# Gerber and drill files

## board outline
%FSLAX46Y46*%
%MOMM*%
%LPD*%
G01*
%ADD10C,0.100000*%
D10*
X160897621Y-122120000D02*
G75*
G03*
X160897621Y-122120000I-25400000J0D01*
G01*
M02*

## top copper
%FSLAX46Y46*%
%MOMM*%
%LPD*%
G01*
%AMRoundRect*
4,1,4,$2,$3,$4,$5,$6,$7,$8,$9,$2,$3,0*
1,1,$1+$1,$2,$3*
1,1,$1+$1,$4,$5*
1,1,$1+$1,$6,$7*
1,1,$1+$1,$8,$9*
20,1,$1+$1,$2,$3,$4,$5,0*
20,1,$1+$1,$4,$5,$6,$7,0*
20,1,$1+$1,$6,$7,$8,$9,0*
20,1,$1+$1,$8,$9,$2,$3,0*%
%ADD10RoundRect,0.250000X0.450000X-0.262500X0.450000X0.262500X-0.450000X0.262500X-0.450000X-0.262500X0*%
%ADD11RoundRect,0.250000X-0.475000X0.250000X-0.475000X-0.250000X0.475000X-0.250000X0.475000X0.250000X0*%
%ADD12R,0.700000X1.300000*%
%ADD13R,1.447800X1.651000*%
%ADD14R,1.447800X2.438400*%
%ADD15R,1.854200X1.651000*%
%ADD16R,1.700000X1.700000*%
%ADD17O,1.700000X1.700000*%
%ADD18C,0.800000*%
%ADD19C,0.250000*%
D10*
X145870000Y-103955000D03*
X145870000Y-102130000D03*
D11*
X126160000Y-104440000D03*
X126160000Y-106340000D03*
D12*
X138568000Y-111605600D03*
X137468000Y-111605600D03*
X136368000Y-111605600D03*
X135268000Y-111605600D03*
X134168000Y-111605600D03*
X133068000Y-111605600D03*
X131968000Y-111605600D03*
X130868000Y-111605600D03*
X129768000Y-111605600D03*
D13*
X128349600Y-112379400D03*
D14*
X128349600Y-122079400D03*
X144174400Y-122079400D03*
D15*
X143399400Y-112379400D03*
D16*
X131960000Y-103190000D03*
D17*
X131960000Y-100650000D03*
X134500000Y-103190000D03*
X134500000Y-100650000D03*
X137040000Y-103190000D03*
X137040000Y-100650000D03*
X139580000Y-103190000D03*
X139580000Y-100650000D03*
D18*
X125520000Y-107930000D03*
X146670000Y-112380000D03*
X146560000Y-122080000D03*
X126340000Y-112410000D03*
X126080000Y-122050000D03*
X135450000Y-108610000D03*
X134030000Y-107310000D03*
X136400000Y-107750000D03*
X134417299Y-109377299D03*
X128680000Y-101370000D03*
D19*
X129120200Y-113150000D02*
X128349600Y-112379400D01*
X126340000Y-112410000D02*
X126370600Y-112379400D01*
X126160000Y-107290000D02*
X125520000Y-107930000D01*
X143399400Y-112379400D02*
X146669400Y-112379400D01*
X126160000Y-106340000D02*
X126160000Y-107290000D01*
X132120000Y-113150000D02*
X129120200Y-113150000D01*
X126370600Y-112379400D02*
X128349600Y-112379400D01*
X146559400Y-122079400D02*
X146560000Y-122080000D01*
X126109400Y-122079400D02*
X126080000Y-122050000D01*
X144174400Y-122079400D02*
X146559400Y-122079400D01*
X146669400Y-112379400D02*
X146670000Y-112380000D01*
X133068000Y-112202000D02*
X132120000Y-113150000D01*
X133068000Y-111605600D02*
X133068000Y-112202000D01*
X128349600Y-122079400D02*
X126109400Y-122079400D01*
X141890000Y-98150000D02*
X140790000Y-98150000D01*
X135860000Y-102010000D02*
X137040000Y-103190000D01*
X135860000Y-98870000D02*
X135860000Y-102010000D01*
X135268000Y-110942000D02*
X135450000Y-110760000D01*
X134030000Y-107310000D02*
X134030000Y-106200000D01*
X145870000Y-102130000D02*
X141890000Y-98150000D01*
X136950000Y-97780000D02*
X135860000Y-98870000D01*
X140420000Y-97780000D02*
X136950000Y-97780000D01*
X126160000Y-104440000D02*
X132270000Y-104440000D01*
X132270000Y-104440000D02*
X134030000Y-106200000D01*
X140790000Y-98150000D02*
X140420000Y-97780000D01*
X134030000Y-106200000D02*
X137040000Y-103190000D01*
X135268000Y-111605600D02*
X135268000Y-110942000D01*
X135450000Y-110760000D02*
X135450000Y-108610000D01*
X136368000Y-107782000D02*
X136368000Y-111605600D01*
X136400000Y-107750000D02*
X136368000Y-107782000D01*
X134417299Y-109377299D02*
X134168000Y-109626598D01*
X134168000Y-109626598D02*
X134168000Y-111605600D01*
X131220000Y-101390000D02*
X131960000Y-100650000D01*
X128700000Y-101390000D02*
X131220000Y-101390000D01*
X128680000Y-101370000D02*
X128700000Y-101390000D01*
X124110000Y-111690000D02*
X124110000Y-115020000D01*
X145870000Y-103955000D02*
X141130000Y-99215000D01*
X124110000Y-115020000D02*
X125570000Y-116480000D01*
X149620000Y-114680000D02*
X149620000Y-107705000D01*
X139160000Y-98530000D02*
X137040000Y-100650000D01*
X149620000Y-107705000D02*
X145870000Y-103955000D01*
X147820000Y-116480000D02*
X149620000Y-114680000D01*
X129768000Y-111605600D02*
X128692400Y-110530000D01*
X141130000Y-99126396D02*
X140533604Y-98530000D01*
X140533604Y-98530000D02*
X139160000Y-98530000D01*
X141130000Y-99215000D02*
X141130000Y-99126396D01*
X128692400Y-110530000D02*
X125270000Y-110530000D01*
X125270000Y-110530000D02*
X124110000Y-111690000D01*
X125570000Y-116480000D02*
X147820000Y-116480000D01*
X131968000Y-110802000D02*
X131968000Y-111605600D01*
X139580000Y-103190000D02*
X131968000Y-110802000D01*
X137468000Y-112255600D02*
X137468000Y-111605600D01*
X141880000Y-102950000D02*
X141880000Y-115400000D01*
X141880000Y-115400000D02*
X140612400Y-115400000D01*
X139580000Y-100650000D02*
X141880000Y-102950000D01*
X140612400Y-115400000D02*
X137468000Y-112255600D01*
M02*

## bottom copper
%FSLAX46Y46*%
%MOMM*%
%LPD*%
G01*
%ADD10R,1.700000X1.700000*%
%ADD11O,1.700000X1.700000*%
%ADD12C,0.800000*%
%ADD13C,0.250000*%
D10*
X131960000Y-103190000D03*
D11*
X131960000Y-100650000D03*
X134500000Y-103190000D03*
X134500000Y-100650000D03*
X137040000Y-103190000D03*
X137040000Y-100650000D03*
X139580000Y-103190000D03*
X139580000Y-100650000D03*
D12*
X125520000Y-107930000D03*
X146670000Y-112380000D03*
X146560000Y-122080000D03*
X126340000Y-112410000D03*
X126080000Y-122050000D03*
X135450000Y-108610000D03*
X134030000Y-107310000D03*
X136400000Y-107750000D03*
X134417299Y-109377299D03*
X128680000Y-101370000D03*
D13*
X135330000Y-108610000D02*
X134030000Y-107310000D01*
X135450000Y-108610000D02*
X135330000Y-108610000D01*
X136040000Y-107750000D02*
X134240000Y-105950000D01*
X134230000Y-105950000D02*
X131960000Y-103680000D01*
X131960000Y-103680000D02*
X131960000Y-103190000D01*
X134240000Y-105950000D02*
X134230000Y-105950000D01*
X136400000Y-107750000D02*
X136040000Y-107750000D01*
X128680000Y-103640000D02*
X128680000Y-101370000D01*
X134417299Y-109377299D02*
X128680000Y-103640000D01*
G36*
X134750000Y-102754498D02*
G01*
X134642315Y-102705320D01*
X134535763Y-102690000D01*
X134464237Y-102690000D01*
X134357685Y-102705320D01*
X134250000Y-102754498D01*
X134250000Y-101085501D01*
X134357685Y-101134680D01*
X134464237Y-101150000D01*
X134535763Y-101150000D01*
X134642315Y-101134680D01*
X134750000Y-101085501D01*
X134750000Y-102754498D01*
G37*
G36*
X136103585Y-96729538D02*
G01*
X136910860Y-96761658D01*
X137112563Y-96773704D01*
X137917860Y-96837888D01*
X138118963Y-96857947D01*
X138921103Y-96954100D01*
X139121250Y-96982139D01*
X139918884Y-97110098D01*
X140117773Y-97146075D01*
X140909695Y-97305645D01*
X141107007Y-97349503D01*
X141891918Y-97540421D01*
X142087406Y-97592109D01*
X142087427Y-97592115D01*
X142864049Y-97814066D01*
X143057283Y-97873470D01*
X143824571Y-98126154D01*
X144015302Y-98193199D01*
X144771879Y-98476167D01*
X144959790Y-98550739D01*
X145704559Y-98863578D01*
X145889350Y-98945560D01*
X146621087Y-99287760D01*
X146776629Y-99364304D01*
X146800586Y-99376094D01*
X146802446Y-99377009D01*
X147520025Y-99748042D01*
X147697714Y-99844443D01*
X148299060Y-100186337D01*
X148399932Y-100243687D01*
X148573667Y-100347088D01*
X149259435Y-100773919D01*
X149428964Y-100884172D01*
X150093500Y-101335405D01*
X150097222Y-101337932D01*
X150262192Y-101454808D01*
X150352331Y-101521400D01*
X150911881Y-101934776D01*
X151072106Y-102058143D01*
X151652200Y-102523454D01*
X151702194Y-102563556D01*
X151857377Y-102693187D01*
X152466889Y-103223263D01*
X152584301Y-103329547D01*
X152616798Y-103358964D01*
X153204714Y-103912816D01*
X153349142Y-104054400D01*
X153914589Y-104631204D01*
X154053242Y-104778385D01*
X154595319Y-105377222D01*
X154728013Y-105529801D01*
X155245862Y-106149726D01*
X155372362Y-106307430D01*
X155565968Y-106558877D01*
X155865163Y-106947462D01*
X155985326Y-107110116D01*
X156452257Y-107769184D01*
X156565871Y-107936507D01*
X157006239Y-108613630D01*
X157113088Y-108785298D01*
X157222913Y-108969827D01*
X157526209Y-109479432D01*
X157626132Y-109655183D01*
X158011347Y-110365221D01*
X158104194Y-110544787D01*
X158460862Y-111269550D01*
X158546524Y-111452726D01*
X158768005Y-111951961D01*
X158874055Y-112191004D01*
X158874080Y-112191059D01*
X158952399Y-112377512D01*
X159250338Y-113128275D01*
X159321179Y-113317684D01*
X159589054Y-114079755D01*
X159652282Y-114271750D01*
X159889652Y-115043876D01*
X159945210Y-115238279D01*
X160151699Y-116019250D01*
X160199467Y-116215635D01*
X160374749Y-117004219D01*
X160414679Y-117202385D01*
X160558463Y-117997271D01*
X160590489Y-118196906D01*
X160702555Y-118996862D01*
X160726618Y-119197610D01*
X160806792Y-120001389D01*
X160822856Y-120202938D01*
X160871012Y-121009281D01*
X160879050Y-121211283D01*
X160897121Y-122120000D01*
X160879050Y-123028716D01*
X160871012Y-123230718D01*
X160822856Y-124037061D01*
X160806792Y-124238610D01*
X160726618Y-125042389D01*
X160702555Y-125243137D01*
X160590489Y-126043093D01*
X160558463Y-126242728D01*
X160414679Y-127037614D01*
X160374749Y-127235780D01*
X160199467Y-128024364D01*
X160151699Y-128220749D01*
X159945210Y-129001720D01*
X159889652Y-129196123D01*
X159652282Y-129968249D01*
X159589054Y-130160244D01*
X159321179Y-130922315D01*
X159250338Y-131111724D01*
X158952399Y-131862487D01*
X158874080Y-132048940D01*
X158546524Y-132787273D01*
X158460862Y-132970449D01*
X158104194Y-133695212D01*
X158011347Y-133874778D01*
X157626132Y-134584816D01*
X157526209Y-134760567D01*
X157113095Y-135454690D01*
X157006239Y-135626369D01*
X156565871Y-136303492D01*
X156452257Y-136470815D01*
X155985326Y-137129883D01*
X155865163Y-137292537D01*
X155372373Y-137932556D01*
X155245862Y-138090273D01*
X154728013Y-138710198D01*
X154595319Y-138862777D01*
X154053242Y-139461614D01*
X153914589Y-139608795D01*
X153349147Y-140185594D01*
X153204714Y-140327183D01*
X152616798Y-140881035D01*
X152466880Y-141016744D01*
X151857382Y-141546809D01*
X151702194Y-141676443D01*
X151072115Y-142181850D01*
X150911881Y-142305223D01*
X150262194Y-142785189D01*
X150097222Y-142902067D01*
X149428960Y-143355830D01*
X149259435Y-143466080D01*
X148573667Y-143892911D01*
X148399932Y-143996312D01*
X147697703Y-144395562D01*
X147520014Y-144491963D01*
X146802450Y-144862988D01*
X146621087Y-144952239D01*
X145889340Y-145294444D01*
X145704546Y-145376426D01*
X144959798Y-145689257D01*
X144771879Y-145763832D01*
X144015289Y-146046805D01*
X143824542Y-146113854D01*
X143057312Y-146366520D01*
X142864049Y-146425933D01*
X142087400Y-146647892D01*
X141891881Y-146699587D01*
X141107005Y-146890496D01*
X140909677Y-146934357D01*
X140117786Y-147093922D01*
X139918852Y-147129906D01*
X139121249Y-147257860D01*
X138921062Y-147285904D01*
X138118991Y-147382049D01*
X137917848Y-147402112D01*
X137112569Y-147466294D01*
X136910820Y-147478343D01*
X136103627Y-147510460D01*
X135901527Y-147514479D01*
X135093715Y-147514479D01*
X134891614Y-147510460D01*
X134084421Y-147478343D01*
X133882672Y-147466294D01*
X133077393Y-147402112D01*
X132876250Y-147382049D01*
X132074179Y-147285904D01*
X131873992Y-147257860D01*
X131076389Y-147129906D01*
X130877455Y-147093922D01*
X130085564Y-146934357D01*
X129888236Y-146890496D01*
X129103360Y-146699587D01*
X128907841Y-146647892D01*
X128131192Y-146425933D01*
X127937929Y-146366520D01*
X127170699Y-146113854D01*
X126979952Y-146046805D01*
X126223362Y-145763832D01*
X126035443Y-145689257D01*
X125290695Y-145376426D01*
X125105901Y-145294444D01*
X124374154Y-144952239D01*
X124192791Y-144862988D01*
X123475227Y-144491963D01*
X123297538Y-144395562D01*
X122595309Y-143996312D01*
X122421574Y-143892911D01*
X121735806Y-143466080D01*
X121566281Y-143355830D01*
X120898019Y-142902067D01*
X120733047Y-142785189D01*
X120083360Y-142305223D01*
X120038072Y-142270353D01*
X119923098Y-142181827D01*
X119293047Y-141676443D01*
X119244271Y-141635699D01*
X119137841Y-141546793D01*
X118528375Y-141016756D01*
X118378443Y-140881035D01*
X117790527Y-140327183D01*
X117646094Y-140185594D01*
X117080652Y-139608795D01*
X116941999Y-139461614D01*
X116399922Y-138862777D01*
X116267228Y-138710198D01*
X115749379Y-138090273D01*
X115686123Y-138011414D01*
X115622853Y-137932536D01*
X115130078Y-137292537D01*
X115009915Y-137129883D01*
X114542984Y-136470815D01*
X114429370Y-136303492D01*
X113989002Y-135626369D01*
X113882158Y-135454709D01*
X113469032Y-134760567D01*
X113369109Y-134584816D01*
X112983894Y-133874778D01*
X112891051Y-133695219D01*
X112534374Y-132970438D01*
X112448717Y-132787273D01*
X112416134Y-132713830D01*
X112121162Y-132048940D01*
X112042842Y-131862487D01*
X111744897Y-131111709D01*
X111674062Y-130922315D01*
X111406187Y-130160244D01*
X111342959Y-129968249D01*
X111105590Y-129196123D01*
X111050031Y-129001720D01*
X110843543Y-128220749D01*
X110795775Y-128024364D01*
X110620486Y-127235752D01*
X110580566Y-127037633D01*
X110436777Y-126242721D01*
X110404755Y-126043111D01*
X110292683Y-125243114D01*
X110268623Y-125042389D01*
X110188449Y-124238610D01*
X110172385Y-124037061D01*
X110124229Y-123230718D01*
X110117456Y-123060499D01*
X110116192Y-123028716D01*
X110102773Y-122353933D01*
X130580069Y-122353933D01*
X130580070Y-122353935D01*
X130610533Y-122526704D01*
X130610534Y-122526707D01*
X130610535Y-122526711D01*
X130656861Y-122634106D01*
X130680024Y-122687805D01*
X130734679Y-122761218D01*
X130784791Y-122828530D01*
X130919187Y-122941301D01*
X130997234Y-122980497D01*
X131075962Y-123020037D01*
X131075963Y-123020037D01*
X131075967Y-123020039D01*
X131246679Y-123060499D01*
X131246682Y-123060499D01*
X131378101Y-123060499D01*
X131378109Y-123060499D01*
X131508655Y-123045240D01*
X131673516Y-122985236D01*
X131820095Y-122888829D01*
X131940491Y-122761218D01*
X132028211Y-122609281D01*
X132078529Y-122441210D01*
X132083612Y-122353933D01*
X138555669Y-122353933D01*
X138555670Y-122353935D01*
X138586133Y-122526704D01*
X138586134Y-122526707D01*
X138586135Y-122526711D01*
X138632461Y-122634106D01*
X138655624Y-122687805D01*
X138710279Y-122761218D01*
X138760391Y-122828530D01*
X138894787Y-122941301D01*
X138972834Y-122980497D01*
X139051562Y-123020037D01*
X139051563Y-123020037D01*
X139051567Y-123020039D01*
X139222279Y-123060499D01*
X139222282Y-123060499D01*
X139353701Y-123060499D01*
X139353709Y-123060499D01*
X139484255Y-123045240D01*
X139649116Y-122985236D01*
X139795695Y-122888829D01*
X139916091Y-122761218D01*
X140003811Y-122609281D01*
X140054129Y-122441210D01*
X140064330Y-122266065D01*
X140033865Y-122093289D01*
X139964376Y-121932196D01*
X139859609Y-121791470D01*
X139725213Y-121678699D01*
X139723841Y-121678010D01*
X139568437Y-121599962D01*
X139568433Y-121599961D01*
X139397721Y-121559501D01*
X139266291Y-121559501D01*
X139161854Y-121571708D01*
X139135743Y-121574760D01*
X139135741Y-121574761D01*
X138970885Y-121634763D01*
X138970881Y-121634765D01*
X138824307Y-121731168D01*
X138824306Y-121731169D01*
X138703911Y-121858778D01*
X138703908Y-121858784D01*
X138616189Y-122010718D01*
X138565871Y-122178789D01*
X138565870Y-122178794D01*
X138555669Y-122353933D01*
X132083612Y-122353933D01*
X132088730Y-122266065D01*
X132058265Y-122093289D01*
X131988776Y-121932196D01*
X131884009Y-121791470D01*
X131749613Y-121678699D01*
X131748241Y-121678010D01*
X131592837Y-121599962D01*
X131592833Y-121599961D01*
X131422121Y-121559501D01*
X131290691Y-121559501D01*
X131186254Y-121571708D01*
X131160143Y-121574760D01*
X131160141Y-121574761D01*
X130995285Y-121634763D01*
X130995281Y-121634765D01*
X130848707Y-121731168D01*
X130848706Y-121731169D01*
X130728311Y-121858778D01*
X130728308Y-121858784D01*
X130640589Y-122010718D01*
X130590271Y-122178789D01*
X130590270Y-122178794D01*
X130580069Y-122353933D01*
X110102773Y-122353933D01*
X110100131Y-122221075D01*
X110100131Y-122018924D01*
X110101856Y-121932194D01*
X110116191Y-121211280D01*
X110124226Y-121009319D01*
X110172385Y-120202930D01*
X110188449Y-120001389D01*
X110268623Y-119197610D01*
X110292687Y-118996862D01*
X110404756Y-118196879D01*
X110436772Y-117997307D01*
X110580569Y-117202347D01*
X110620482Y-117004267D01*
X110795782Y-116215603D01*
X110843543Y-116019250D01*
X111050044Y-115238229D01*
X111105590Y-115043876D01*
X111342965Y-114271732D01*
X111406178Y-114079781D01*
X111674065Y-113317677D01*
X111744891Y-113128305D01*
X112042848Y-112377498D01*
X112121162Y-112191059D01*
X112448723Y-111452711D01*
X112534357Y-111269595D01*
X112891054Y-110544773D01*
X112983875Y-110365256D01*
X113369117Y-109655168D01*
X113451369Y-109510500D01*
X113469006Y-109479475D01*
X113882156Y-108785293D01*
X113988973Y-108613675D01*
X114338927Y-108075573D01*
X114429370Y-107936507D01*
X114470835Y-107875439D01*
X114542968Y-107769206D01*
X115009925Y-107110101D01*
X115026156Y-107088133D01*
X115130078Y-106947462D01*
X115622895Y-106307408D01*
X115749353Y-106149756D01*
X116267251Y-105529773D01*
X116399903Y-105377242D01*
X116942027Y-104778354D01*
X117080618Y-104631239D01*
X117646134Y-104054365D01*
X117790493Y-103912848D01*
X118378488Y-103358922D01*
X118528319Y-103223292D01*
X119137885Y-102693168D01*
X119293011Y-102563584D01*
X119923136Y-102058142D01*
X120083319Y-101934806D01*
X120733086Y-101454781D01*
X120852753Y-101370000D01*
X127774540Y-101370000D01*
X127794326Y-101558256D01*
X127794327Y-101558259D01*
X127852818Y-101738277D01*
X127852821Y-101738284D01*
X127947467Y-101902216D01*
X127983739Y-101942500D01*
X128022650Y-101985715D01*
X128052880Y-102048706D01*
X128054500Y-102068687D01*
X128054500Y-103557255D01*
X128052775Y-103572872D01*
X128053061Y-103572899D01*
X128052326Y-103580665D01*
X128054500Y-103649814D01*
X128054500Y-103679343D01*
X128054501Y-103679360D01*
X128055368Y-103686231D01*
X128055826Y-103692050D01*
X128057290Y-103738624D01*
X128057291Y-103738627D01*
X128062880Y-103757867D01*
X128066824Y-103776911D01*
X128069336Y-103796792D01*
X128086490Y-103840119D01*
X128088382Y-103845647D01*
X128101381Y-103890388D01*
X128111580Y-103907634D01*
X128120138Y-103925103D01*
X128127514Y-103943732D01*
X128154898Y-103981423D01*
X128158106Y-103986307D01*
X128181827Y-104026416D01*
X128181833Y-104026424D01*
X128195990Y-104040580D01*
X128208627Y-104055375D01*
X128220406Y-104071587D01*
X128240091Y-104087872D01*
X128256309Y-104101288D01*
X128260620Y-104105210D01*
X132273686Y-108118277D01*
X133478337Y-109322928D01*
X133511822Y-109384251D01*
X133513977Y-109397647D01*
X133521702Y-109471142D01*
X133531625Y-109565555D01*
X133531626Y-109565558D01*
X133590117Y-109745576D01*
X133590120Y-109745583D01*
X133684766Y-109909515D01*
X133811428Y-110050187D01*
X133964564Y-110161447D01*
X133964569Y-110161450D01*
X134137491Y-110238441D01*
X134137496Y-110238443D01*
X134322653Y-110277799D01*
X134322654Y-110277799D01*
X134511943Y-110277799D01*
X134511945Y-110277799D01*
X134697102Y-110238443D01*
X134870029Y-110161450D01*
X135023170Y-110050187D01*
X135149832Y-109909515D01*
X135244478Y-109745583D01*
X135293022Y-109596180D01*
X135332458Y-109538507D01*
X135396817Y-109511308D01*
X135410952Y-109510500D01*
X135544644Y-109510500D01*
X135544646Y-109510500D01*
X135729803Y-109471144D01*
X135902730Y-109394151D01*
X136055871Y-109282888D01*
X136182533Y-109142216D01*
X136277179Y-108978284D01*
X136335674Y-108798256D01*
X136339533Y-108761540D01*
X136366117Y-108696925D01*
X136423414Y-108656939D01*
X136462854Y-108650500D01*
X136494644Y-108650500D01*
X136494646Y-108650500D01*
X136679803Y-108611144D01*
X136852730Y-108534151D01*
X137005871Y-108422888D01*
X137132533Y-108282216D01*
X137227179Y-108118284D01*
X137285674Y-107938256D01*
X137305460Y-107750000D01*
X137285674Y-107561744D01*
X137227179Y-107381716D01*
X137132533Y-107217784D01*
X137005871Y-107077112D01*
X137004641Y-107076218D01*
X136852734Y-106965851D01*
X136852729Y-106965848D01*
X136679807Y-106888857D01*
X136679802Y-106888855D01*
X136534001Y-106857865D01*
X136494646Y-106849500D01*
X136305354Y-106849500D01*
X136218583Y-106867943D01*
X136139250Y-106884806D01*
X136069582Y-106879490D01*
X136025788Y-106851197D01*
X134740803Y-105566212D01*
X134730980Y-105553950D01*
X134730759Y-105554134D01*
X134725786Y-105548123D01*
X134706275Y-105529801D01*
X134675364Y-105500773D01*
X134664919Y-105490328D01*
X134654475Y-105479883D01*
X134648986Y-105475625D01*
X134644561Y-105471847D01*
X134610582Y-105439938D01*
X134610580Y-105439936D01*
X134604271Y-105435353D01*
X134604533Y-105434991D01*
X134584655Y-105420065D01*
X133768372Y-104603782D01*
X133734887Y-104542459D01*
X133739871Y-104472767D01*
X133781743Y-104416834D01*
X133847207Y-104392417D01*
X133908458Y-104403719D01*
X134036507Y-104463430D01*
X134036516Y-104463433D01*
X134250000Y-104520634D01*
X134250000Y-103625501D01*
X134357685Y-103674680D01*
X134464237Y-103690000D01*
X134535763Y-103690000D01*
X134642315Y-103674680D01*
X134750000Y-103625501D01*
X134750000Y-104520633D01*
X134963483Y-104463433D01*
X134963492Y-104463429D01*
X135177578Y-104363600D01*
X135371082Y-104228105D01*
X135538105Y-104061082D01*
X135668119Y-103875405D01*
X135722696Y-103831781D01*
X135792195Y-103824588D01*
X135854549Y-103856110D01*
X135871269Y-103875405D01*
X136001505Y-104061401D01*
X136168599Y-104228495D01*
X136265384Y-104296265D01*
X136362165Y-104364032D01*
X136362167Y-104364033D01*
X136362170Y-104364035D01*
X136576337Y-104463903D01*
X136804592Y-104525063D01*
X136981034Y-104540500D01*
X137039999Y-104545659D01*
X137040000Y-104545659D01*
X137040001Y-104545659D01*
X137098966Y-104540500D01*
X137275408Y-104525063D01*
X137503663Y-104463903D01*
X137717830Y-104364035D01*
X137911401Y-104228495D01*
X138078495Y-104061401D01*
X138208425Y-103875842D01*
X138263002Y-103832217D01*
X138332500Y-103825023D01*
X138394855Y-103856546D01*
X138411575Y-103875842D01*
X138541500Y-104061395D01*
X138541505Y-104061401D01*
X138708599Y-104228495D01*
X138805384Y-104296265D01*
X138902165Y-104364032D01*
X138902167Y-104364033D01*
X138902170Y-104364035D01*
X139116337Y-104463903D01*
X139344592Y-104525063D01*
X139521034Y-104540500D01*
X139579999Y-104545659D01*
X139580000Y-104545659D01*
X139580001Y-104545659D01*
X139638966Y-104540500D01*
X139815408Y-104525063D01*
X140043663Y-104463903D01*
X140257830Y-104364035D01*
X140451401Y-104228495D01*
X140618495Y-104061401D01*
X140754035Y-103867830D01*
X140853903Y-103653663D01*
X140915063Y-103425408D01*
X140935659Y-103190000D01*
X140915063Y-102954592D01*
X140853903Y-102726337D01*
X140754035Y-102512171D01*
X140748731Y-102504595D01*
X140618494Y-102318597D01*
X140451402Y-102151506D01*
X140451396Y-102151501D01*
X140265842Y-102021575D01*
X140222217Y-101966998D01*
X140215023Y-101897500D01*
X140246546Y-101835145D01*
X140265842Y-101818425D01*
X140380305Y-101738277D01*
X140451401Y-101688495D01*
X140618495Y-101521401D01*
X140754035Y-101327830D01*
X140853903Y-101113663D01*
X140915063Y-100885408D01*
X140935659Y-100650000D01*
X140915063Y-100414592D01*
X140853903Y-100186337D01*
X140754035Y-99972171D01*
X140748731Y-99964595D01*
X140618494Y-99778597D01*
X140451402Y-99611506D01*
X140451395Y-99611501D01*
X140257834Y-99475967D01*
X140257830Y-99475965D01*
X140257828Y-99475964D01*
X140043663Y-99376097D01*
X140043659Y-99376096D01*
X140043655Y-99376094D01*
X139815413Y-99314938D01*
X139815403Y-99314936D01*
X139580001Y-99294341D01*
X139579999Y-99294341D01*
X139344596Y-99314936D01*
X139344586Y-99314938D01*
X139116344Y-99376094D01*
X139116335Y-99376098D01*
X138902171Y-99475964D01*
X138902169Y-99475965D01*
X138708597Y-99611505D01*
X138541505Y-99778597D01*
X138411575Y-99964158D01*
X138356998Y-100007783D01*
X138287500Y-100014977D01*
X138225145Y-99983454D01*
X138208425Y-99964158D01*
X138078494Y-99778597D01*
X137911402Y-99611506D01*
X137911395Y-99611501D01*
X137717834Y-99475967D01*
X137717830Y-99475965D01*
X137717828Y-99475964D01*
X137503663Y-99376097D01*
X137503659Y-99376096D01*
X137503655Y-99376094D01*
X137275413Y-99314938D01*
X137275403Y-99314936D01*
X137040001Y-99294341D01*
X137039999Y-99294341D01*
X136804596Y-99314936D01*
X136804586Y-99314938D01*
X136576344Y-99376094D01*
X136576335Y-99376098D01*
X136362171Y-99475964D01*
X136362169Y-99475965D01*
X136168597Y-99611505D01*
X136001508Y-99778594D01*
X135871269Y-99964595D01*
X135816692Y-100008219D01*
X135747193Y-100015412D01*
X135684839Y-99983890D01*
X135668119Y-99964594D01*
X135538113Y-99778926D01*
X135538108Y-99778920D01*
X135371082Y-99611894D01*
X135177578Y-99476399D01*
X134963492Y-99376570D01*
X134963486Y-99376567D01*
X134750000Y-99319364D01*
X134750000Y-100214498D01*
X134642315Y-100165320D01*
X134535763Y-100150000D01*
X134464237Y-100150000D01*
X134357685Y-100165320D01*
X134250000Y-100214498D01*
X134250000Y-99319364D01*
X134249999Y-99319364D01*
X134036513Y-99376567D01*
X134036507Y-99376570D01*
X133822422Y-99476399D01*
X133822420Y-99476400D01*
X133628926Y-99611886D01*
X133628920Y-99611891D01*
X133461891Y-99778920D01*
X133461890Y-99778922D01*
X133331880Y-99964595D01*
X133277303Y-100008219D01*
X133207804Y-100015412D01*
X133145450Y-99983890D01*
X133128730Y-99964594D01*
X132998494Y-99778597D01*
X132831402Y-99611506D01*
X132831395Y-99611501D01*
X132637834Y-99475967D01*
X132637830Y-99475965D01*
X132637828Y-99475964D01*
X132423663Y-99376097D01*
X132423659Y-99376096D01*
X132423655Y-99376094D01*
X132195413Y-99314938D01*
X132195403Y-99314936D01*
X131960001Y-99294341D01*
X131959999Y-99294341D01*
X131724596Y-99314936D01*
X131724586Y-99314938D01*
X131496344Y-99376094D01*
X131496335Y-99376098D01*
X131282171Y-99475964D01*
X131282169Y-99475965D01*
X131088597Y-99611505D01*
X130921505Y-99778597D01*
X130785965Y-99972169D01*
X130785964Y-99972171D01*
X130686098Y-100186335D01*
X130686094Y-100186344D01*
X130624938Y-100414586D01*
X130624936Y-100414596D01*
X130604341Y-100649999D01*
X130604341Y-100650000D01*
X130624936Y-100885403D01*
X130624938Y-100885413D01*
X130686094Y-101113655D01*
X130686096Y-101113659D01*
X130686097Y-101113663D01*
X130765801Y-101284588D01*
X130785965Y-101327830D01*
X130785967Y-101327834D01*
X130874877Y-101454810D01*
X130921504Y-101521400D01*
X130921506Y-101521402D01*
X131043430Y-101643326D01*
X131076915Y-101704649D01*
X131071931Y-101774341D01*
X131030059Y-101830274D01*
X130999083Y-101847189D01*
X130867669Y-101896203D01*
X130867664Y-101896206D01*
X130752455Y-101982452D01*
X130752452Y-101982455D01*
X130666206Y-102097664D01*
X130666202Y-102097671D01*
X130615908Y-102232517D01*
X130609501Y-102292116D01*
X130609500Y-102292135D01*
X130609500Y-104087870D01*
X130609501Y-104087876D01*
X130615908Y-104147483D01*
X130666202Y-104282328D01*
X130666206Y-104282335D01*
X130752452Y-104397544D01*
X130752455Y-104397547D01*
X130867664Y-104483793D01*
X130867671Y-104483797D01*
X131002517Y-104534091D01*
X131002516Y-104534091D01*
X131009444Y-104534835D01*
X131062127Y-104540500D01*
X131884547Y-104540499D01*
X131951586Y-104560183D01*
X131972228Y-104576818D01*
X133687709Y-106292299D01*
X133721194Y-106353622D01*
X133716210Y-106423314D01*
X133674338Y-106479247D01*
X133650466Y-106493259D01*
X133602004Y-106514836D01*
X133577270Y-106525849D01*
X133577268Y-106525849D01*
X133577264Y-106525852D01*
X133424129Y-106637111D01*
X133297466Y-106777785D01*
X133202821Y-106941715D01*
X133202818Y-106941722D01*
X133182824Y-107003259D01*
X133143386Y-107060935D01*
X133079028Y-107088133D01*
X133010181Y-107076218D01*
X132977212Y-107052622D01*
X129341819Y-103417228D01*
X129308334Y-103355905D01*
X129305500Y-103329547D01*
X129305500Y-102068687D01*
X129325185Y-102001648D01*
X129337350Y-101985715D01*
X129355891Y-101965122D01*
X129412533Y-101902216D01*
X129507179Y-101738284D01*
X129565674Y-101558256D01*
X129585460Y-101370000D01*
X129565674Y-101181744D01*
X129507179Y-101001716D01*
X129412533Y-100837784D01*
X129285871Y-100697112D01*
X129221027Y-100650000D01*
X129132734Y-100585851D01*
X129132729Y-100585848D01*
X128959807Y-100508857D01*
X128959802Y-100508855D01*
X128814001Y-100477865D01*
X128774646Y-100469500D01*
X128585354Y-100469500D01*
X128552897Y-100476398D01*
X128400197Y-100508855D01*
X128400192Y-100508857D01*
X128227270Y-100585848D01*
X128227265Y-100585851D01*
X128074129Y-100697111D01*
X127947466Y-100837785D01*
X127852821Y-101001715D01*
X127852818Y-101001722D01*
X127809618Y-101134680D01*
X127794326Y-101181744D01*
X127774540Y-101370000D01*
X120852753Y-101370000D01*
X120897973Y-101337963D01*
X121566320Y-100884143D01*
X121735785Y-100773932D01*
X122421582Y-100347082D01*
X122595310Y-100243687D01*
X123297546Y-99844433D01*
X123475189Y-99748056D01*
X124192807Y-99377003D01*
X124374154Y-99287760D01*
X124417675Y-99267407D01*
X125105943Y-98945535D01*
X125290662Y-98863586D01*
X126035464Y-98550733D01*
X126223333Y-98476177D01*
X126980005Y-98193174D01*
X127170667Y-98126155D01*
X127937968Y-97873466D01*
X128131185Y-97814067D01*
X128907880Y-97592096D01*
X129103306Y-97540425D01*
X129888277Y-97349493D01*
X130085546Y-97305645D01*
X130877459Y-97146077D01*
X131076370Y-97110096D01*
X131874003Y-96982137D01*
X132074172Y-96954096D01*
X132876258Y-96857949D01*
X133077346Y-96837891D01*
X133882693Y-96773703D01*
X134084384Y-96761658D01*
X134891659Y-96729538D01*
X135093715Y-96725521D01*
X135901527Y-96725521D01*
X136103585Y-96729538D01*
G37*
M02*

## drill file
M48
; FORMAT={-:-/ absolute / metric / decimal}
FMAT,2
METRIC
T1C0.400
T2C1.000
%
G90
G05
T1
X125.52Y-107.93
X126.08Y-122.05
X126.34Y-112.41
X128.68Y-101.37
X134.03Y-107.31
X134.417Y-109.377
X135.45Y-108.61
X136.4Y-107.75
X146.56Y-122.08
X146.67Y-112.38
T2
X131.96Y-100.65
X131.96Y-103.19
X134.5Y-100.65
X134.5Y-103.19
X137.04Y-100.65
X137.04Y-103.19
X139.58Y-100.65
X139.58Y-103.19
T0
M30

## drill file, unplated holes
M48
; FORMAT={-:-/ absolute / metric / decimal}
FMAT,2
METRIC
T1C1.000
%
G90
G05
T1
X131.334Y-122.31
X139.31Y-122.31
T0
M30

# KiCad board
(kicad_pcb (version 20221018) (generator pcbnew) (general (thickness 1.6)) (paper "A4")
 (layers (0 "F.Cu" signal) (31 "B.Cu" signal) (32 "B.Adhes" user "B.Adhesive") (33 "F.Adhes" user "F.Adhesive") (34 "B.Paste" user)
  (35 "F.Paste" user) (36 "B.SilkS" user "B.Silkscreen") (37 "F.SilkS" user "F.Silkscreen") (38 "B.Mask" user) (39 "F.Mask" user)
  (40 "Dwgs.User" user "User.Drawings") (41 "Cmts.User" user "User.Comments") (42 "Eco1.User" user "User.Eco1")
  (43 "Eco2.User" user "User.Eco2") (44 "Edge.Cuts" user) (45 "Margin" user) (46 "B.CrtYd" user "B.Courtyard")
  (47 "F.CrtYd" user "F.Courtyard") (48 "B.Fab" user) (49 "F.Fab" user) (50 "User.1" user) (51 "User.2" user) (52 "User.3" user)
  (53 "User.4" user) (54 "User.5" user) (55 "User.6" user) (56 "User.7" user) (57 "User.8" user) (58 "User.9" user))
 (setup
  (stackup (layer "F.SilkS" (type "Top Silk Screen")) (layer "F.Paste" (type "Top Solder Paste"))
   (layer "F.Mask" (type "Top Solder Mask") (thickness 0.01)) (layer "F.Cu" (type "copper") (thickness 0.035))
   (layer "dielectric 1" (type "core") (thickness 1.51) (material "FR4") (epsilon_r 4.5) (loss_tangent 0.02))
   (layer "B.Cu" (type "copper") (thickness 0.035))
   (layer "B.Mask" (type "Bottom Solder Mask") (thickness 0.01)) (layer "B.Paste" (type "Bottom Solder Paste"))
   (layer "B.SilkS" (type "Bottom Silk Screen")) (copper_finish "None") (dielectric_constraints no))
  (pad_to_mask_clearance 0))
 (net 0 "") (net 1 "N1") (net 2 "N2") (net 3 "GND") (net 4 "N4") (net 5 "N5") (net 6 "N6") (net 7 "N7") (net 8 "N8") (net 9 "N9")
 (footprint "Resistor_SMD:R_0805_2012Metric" (layer "F.Cu") (at 145.87 103.0425 90)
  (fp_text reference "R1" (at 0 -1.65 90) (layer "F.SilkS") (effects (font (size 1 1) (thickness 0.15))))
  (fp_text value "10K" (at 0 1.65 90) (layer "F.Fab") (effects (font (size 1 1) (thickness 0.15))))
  (pad "1" smd roundrect (at -0.9125 0 90) (size 1.025 1.4) (layers "F.Cu" "F.Paste" "F.Mask") (roundrect_rratio 0.243902439) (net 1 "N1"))
  (pad "2" smd roundrect (at 0.9125 0 90) (size 1.025 1.4) (layers "F.Cu" "F.Paste" "F.Mask") (roundrect_rratio 0.243902439) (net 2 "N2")))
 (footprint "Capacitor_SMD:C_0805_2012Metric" (layer "F.Cu") (at 126.16 105.39 -90)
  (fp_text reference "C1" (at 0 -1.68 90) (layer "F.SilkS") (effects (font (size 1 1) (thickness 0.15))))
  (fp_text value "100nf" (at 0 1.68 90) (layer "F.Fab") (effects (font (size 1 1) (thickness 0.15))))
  (pad "1" smd roundrect (at -0.95 0 270) (size 1 1.45) (layers "F.Cu" "F.Paste" "F.Mask") (roundrect_rratio 0.25) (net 2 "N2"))
  (pad "2" smd roundrect (at 0.95 0 270) (size 1 1.45) (layers "F.Cu" "F.Paste" "F.Mask") (roundrect_rratio 0.25) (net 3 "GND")))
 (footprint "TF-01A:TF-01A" (layer "F.Cu") (at 136.3382 118.7794)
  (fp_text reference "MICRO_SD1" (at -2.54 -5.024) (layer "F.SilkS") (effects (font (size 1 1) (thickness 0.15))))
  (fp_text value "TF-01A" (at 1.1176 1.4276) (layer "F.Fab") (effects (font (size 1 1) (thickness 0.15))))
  (pad "" np_thru_hole circle (at -5.0038 3.5306) (size 0.999997 0.999997) (drill 0.999997) (layers "*.Cu" "*.Mask"))
  (pad "" np_thru_hole circle (at 2.9718 3.5306) (size 0.999997 0.999997) (drill 0.999997) (layers "*.Cu" "*.Mask"))
  (pad "1" smd rect (at 2.2298 -7.1738) (size 0.7 1.3) (layers "F.Cu" "F.Paste" "F.Mask") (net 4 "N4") (solder_mask_margin 0.102))
  (pad "2" smd rect (at 1.1298 -7.1738) (size 0.7 1.3) (layers "F.Cu" "F.Paste" "F.Mask") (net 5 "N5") (solder_mask_margin 0.102))
  (pad "3" smd rect (at 0.0298 -7.1738) (size 0.7 1.3) (layers "F.Cu" "F.Paste" "F.Mask") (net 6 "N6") (solder_mask_margin 0.102))
  (pad "4" smd rect (at -1.0702 -7.1738) (size 0.7 1.3) (layers "F.Cu" "F.Paste" "F.Mask") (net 2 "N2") (solder_mask_margin 0.102))
  (pad "5" smd rect (at -2.1702 -7.1738) (size 0.7 1.3) (layers "F.Cu" "F.Paste" "F.Mask") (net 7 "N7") (solder_mask_margin 0.102))
  (pad "6" smd rect (at -3.2702 -7.1738) (size 0.7 1.3) (layers "F.Cu" "F.Paste" "F.Mask") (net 3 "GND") (solder_mask_margin 0.102))
  (pad "7" smd rect (at -4.3702 -7.1738) (size 0.7 1.3) (layers "F.Cu" "F.Paste" "F.Mask") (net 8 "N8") (solder_mask_margin 0.102))
  (pad "8" smd rect (at -5.4702 -7.1738) (size 0.7 1.3) (layers "F.Cu" "F.Paste" "F.Mask") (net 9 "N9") (solder_mask_margin 0.102))
  (pad "CD1" smd rect (at -6.5702 -7.1738) (size 0.7 1.3) (layers "F.Cu" "F.Paste" "F.Mask") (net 1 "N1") (solder_mask_margin 0.102))
  (pad "MP1" smd rect (at -7.9886 -6.4) (size 1.4478 1.651) (layers "F.Cu" "F.Paste" "F.Mask") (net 3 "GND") (solder_mask_margin 0.102))
  (pad "MP2" smd rect (at -7.9886 3.3) (size 1.4478 2.4384) (layers "F.Cu" "F.Paste" "F.Mask") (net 3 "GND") (solder_mask_margin 0.102))
  (pad "MP3" smd rect (at 7.8362 3.3) (size 1.4478 2.4384) (layers "F.Cu" "F.Paste" "F.Mask") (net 3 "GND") (solder_mask_margin 0.102))
  (pad "MP4" smd rect (at 7.0612 -6.4) (size 1.8542 1.651) (layers "F.Cu" "F.Paste" "F.Mask") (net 3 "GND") (solder_mask_margin 0.102)))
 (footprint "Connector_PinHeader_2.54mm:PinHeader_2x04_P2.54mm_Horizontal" (layer "F.Cu") (at 131.96 103.19 90)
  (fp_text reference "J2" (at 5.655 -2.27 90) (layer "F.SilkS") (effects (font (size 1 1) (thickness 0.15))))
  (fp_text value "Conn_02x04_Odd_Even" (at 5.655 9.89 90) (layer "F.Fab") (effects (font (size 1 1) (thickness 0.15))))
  (pad "1" thru_hole rect (at 0 0 90) (size 1.7 1.7) (drill 1) (layers "*.Cu" "*.Mask") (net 6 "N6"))
  (pad "2" thru_hole oval (at 2.54 0 90) (size 1.7 1.7) (drill 1) (layers "*.Cu" "*.Mask") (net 7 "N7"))
  (pad "3" thru_hole oval (at 0 2.54 90) (size 1.7 1.7) (drill 1) (layers "*.Cu" "*.Mask") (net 3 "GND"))
  (pad "4" thru_hole oval (at 2.54 2.54 90) (size 1.7 1.7) (drill 1) (layers "*.Cu" "*.Mask") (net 3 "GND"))
  (pad "5" thru_hole oval (at 0 5.08 90) (size 1.7 1.7) (drill 1) (layers "*.Cu" "*.Mask") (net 2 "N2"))
  (pad "6" thru_hole oval (at 2.54 5.08 90) (size 1.7 1.7) (drill 1) (layers "*.Cu" "*.Mask") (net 1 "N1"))
  (pad "7" thru_hole oval (at 0 7.62 90) (size 1.7 1.7) (drill 1) (layers "*.Cu" "*.Mask") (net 8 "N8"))
  (pad "8" thru_hole oval (at 2.54 7.62 90) (size 1.7 1.7) (drill 1) (layers "*.Cu" "*.Mask") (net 5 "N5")))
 (gr_circle (center 135.497621 122.12) (end 160.897621 122.12) (stroke (width 0.1) (type default)) (fill none) (layer "Edge.Cuts"))
 (segment (start 129.1202 113.15) (end 128.3496 112.3794) (width 0.25) (layer "F.Cu") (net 3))
 (segment (start 126.34 112.41) (end 126.3706 112.3794) (width 0.25) (layer "F.Cu") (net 3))
 (segment (start 126.16 107.29) (end 125.52 107.93) (width 0.25) (layer "F.Cu") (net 3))
 (segment (start 143.3994 112.3794) (end 146.6694 112.3794) (width 0.25) (layer "F.Cu") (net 3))
 (segment (start 126.16 106.34) (end 126.16 107.29) (width 0.25) (layer "F.Cu") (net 3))
 (segment (start 132.12 113.15) (end 129.1202 113.15) (width 0.25) (layer "F.Cu") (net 3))
 (segment (start 126.3706 112.3794) (end 128.3496 112.3794) (width 0.25) (layer "F.Cu") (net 3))
 (segment (start 146.5594 122.0794) (end 146.56 122.08) (width 0.25) (layer "F.Cu") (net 3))
 (segment (start 126.1094 122.0794) (end 126.08 122.05) (width 0.25) (layer "F.Cu") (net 3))
 (segment (start 144.1744 122.0794) (end 146.5594 122.0794) (width 0.25) (layer "F.Cu") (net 3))
 (segment (start 146.6694 112.3794) (end 146.67 112.38) (width 0.25) (layer "F.Cu") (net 3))
 (segment (start 133.068 112.202) (end 132.12 113.15) (width 0.25) (layer "F.Cu") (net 3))
 (segment (start 133.068 111.6056) (end 133.068 112.202) (width 0.25) (layer "F.Cu") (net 3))
 (segment (start 128.3496 122.0794) (end 126.1094 122.0794) (width 0.25) (layer "F.Cu") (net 3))
 (via (at 125.52 107.93) (size 0.8) (drill 0.4) (layers "F.Cu" "B.Cu") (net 3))
 (via (at 146.67 112.38) (size 0.8) (drill 0.4) (layers "F.Cu" "B.Cu") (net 3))
 (via (at 146.56 122.08) (size 0.8) (drill 0.4) (layers "F.Cu" "B.Cu") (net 3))
 (via (at 126.34 112.41) (size 0.8) (drill 0.4) (layers "F.Cu" "B.Cu") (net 3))
 (via (at 126.08 122.05) (size 0.8) (drill 0.4) (layers "F.Cu" "B.Cu") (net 3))
 (segment (start 141.89 98.15) (end 140.79 98.15) (width 0.25) (layer "F.Cu") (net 2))
 (segment (start 135.86 102.01) (end 137.04 103.19) (width 0.25) (layer "F.Cu") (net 2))
 (segment (start 135.86 98.87) (end 135.86 102.01) (width 0.25) (layer "F.Cu") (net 2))
 (segment (start 135.268 110.942) (end 135.45 110.76) (width 0.25) (layer "F.Cu") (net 2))
 (segment (start 134.03 107.31) (end 134.03 106.2) (width 0.25) (layer "F.Cu") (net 2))
 (segment (start 145.87 102.13) (end 141.89 98.15) (width 0.25) (layer "F.Cu") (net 2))
 (segment (start 136.95 97.78) (end 135.86 98.87) (width 0.25) (layer "F.Cu") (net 2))
 (segment (start 140.42 97.78) (end 136.95 97.78) (width 0.25) (layer "F.Cu") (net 2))
 (segment (start 126.16 104.44) (end 132.27 104.44) (width 0.25) (layer "F.Cu") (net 2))
 (segment (start 132.27 104.44) (end 134.03 106.2) (width 0.25) (layer "F.Cu") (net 2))
 (segment (start 140.79 98.15) (end 140.42 97.78) (width 0.25) (layer "F.Cu") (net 2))
 (segment (start 134.03 106.2) (end 137.04 103.19) (width 0.25) (layer "F.Cu") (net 2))
 (segment (start 135.268 111.6056) (end 135.268 110.942) (width 0.25) (layer "F.Cu") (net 2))
 (segment (start 135.45 110.76) (end 135.45 108.61) (width 0.25) (layer "F.Cu") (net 2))
 (via (at 135.45 108.61) (size 0.8) (drill 0.4) (layers "F.Cu" "B.Cu") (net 2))
 (via (at 134.03 107.31) (size 0.8) (drill 0.4) (layers "F.Cu" "B.Cu") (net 2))
 (segment (start 135.33 108.61) (end 134.03 107.31) (width 0.25) (layer "B.Cu") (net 2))
 (segment (start 135.45 108.61) (end 135.33 108.61) (width 0.25) (layer "B.Cu") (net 2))
 (segment (start 136.368 107.782) (end 136.368 111.6056) (width 0.25) (layer "F.Cu") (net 6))
 (segment (start 136.4 107.75) (end 136.368 107.782) (width 0.25) (layer "F.Cu") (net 6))
 (via (at 136.4 107.75) (size 0.8) (drill 0.4) (layers "F.Cu" "B.Cu") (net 6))
 (segment (start 136.04 107.75) (end 134.24 105.95) (width 0.25) (layer "B.Cu") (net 6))
 (segment (start 134.23 105.95) (end 131.96 103.68) (width 0.25) (layer "B.Cu") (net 6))
 (segment (start 131.96 103.68) (end 131.96 103.19) (width 0.25) (layer "B.Cu") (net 6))
 (segment (start 134.24 105.95) (end 134.23 105.95) (width 0.25) (layer "B.Cu") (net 6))
 (segment (start 136.4 107.75) (end 136.04 107.75) (width 0.25) (layer "B.Cu") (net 6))
 (segment (start 134.417299 109.377299) (end 134.168 109.626598) (width 0.25) (layer "F.Cu") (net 7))
 (segment (start 134.168 109.626598) (end 134.168 111.6056) (width 0.25) (layer "F.Cu") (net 7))
 (segment (start 131.22 101.39) (end 131.96 100.65) (width 0.25) (layer "F.Cu") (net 7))
 (segment (start 128.7 101.39) (end 131.22 101.39) (width 0.25) (layer "F.Cu") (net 7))
 (segment (start 128.68 101.37) (end 128.7 101.39) (width 0.25) (layer "F.Cu") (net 7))
 (via (at 134.417299 109.377299) (size 0.8) (drill 0.4) (layers "F.Cu" "B.Cu") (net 7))
 (via (at 128.68 101.37) (size 0.8) (drill 0.4) (layers "F.Cu" "B.Cu") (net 7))
 (segment (start 128.68 103.64) (end 128.68 101.37) (width 0.25) (layer "B.Cu") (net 7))
 (segment (start 134.417299 109.377299) (end 128.68 103.64) (width 0.25) (layer "B.Cu") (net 7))
 (segment (start 124.11 111.69) (end 124.11 115.02) (width 0.25) (layer "F.Cu") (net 1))
 (segment (start 145.87 103.955) (end 141.13 99.215) (width 0.25) (layer "F.Cu") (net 1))
 (segment (start 124.11 115.02) (end 125.57 116.48) (width 0.25) (layer "F.Cu") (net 1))
 (segment (start 149.62 114.68) (end 149.62 107.705) (width 0.25) (layer "F.Cu") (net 1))
 (segment (start 139.16 98.53) (end 137.04 100.65) (width 0.25) (layer "F.Cu") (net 1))
 (segment (start 149.62 107.705) (end 145.87 103.955) (width 0.25) (layer "F.Cu") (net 1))
 (segment (start 147.82 116.48) (end 149.62 114.68) (width 0.25) (layer "F.Cu") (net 1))
 (segment (start 129.768 111.6056) (end 128.6924 110.53) (width 0.25) (layer "F.Cu") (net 1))
 (segment (start 141.13 99.126396) (end 140.533604 98.53) (width 0.25) (layer "F.Cu") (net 1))
 (segment (start 140.533604 98.53) (end 139.16 98.53) (width 0.25) (layer "F.Cu") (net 1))
 (segment (start 141.13 99.215) (end 141.13 99.126396) (width 0.25) (layer "F.Cu") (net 1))
 (segment (start 128.6924 110.53) (end 125.27 110.53) (width 0.25) (layer "F.Cu") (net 1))
 (segment (start 125.27 110.53) (end 124.11 111.69) (width 0.25) (layer "F.Cu") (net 1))
 (segment (start 125.57 116.48) (end 147.82 116.48) (width 0.25) (layer "F.Cu") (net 1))
 (segment (start 131.968 110.802) (end 131.968 111.6056) (width 0.25) (layer "F.Cu") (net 8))
 (segment (start 139.58 103.19) (end 131.968 110.802) (width 0.25) (layer "F.Cu") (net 8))
 (segment (start 137.468 112.2556) (end 137.468 111.6056) (width 0.25) (layer "F.Cu") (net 5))
 (segment (start 141.88 102.95) (end 141.88 115.4) (width 0.25) (layer "F.Cu") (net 5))
 (segment (start 141.88 115.4) (end 140.6124 115.4) (width 0.25) (layer "F.Cu") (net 5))
 (segment (start 139.58 100.65) (end 141.88 102.95) (width 0.25) (layer "F.Cu") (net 5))
 (segment (start 140.6124 115.4) (end 137.468 112.2556) (width 0.25) (layer "F.Cu") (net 5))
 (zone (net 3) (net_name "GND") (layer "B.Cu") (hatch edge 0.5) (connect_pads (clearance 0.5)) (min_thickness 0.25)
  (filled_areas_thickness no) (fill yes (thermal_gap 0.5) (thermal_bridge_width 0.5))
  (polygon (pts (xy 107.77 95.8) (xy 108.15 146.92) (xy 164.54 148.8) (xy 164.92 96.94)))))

